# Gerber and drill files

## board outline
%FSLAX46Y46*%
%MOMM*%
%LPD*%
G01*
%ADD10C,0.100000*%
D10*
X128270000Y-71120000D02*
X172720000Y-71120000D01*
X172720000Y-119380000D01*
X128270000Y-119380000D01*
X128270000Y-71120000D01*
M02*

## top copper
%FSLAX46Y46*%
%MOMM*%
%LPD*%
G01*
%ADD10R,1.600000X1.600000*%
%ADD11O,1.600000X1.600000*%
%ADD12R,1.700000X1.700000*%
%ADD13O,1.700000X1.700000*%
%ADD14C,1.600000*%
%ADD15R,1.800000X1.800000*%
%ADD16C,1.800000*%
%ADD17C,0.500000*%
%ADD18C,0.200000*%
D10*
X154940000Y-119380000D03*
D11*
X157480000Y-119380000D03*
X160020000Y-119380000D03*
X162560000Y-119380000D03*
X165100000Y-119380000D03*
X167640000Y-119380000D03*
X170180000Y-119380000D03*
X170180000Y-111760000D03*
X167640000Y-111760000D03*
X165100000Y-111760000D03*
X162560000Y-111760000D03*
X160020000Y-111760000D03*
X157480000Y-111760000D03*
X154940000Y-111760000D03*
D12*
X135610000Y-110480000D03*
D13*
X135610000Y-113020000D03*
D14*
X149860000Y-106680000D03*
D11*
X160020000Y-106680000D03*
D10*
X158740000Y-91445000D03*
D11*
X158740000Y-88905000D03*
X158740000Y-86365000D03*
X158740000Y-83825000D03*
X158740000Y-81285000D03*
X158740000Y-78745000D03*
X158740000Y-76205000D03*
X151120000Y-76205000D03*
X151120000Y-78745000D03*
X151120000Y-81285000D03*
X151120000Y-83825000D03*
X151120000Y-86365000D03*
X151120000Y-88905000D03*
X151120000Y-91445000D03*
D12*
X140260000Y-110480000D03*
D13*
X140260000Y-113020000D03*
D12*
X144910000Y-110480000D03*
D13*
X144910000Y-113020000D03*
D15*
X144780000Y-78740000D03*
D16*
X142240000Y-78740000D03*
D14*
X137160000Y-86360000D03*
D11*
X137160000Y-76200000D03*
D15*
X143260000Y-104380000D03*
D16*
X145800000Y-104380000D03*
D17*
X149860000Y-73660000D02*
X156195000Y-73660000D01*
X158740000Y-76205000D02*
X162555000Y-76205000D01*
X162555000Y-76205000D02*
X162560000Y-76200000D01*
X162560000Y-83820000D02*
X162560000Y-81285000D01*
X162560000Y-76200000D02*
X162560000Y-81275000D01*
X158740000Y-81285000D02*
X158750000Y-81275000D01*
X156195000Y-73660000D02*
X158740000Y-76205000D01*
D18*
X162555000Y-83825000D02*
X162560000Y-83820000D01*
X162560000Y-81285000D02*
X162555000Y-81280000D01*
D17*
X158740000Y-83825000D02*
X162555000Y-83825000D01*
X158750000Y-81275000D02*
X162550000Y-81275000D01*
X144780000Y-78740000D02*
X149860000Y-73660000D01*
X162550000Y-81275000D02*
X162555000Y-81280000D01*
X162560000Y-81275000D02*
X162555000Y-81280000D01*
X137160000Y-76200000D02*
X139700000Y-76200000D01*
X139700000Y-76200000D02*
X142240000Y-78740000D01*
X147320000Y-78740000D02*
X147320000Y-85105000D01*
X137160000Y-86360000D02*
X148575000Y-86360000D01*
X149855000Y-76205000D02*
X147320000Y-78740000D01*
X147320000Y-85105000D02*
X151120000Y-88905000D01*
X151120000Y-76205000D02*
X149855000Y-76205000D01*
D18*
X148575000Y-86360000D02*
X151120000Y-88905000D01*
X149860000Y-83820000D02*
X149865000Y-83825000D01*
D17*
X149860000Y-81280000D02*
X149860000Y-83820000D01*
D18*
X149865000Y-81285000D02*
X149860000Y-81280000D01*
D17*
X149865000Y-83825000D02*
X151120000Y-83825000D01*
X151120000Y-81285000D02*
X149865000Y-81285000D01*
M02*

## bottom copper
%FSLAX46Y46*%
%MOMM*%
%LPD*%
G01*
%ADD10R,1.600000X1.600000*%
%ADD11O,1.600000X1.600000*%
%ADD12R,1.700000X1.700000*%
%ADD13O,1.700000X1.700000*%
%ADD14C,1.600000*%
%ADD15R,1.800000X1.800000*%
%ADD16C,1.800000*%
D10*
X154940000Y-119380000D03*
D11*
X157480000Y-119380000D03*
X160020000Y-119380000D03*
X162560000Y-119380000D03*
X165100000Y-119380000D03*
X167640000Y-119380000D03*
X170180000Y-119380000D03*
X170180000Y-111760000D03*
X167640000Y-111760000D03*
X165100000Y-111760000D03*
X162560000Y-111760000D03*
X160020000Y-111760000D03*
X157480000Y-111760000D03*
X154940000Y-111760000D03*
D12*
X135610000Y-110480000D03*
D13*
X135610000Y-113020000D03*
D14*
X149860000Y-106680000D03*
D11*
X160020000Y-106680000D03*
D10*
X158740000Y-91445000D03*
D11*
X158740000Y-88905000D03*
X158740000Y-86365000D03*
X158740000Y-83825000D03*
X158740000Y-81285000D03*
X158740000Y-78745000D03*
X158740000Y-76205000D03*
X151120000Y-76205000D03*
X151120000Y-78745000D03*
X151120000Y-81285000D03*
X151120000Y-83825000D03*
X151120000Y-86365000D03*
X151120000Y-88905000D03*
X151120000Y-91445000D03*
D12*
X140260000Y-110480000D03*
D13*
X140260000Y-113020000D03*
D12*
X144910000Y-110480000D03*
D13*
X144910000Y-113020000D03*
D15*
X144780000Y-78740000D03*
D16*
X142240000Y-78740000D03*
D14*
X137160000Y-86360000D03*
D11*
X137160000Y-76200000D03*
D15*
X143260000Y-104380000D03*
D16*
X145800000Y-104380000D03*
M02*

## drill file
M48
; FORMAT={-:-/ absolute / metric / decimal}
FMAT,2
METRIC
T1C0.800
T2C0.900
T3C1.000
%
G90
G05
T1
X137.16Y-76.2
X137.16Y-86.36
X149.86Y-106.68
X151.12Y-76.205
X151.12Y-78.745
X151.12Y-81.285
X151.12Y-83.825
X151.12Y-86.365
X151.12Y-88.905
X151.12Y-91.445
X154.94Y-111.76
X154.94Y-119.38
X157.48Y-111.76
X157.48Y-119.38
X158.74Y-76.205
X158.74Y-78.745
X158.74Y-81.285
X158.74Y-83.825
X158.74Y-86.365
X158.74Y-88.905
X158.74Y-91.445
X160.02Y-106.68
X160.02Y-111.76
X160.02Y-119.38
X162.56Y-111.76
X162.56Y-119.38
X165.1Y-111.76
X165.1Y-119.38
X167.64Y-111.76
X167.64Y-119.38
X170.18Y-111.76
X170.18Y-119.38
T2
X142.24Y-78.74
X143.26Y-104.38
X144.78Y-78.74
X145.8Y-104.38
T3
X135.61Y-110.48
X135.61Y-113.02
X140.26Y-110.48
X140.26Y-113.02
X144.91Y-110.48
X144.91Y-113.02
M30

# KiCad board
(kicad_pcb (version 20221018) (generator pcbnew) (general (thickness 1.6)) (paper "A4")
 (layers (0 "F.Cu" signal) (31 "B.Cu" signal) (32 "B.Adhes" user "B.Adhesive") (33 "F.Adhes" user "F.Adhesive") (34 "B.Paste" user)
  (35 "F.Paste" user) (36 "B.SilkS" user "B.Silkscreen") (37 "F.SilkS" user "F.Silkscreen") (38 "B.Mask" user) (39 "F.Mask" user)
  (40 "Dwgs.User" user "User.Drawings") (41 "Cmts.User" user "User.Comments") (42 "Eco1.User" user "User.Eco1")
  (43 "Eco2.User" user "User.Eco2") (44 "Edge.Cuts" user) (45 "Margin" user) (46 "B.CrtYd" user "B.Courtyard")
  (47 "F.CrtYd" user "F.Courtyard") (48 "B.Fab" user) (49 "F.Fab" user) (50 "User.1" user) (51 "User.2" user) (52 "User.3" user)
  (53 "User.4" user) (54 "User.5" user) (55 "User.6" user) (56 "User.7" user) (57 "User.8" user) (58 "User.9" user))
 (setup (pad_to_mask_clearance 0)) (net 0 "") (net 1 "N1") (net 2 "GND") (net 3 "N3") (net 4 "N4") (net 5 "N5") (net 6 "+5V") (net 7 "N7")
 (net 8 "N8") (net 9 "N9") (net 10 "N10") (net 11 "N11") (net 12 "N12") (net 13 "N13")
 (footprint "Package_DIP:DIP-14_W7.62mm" (layer "F.Cu") (at 154.94 119.38 90)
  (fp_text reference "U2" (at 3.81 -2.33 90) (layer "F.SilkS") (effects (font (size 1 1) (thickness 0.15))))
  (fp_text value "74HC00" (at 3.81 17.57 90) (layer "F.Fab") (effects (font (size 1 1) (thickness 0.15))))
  (pad "1" thru_hole rect (at 0 0 90) (size 1.6 1.6) (drill 0.8) (layers "*.Cu" "*.Mask") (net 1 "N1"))
  (pad "2" thru_hole oval (at 0 2.54 90) (size 1.6 1.6) (drill 0.8) (layers "*.Cu" "*.Mask") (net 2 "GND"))
  (pad "3" thru_hole oval (at 0 5.08 90) (size 1.6 1.6) (drill 0.8) (layers "*.Cu" "*.Mask") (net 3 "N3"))
  (pad "4" thru_hole oval (at 0 7.62 90) (size 1.6 1.6) (drill 0.8) (layers "*.Cu" "*.Mask") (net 2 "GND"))
  (pad "5" thru_hole oval (at 0 10.16 90) (size 1.6 1.6) (drill 0.8) (layers "*.Cu" "*.Mask") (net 2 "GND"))
  (pad "6" thru_hole oval (at 0 12.7 90) (size 1.6 1.6) (drill 0.8) (layers "*.Cu" "*.Mask") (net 1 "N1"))
  (pad "7" thru_hole oval (at 0 15.24 90) (size 1.6 1.6) (drill 0.8) (layers "*.Cu" "*.Mask") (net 2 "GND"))
  (pad "8" thru_hole oval (at 7.62 15.24 90) (size 1.6 1.6) (drill 0.8) (layers "*.Cu" "*.Mask") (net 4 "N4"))
  (pad "9" thru_hole oval (at 7.62 12.7 90) (size 1.6 1.6) (drill 0.8) (layers "*.Cu" "*.Mask") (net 1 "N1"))
  (pad "10" thru_hole oval (at 7.62 10.16 90) (size 1.6 1.6) (drill 0.8) (layers "*.Cu" "*.Mask") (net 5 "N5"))
  (pad "11" thru_hole oval (at 7.62 7.62 90) (size 1.6 1.6) (drill 0.8) (layers "*.Cu" "*.Mask") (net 5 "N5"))
  (pad "12" thru_hole oval (at 7.62 5.08 90) (size 1.6 1.6) (drill 0.8) (layers "*.Cu" "*.Mask") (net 3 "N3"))
  (pad "13" thru_hole oval (at 7.62 2.54 90) (size 1.6 1.6) (drill 0.8) (layers "*.Cu" "*.Mask") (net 4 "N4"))
  (pad "14" thru_hole oval (at 7.62 0 90) (size 1.6 1.6) (drill 0.8) (layers "*.Cu" "*.Mask") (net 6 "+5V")))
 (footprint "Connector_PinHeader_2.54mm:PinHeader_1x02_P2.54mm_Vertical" (layer "F.Cu") (at 135.61 110.48)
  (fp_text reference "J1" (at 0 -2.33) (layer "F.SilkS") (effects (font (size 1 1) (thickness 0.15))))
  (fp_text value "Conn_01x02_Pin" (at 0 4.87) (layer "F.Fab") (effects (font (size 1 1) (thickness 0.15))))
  (pad "1" thru_hole rect (at 0 0) (size 1.7 1.7) (drill 1) (layers "*.Cu" "*.Mask") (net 6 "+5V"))
  (pad "2" thru_hole oval (at 0 2.54) (size 1.7 1.7) (drill 1) (layers "*.Cu" "*.Mask") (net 2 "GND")))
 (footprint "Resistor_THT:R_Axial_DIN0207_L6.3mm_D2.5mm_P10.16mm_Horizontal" (layer "F.Cu") (at 149.86 106.68)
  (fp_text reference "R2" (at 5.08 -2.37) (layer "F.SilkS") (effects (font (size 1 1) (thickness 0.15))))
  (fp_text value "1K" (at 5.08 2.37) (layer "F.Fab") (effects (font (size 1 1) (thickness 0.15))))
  (pad "1" thru_hole circle (at 0 0) (size 1.6 1.6) (drill 0.8) (layers "*.Cu" "*.Mask") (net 4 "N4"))
  (pad "2" thru_hole oval (at 10.16 0) (size 1.6 1.6) (drill 0.8) (layers "*.Cu" "*.Mask") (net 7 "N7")))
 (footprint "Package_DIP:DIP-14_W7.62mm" (layer "F.Cu") (at 158.74 91.445 180)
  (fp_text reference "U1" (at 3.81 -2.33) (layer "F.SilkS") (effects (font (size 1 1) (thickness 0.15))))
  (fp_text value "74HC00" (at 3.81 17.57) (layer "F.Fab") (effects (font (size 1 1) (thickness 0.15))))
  (pad "1" thru_hole rect (at 0 0 180) (size 1.6 1.6) (drill 0.8) (layers "*.Cu" "*.Mask") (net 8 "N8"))
  (pad "2" thru_hole oval (at 0 2.54 180) (size 1.6 1.6) (drill 0.8) (layers "*.Cu" "*.Mask") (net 2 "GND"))
  (pad "3" thru_hole oval (at 0 5.08 180) (size 1.6 1.6) (drill 0.8) (layers "*.Cu" "*.Mask") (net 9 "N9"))
  (pad "4" thru_hole oval (at 0 7.62 180) (size 1.6 1.6) (drill 0.8) (layers "*.Cu" "*.Mask") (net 2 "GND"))
  (pad "5" thru_hole oval (at 0 10.16 180) (size 1.6 1.6) (drill 0.8) (layers "*.Cu" "*.Mask") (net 2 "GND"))
  (pad "6" thru_hole oval (at 0 12.7 180) (size 1.6 1.6) (drill 0.8) (layers "*.Cu" "*.Mask") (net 8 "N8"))
  (pad "7" thru_hole oval (at 0 15.24 180) (size 1.6 1.6) (drill 0.8) (layers "*.Cu" "*.Mask") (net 2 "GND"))
  (pad "8" thru_hole oval (at 7.62 15.24 180) (size 1.6 1.6) (drill 0.8) (layers "*.Cu" "*.Mask") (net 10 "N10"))
  (pad "9" thru_hole oval (at 7.62 12.7 180) (size 1.6 1.6) (drill 0.8) (layers "*.Cu" "*.Mask") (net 8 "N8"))
  (pad "10" thru_hole oval (at 7.62 10.16 180) (size 1.6 1.6) (drill 0.8) (layers "*.Cu" "*.Mask") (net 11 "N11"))
  (pad "11" thru_hole oval (at 7.62 7.62 180) (size 1.6 1.6) (drill 0.8) (layers "*.Cu" "*.Mask") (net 11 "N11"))
  (pad "12" thru_hole oval (at 7.62 5.08 180) (size 1.6 1.6) (drill 0.8) (layers "*.Cu" "*.Mask") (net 9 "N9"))
  (pad "13" thru_hole oval (at 7.62 2.54 180) (size 1.6 1.6) (drill 0.8) (layers "*.Cu" "*.Mask") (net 10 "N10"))
  (pad "14" thru_hole oval (at 7.62 0 180) (size 1.6 1.6) (drill 0.8) (layers "*.Cu" "*.Mask") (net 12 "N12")))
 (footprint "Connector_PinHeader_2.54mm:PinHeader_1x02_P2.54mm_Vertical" (layer "F.Cu") (at 140.26 110.48)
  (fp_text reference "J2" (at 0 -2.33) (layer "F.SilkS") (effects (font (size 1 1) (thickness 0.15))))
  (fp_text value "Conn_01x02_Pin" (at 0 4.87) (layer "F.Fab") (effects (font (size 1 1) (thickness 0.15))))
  (pad "1" thru_hole rect (at 0 0) (size 1.7 1.7) (drill 1) (layers "*.Cu" "*.Mask") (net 6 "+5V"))
  (pad "2" thru_hole oval (at 0 2.54) (size 1.7 1.7) (drill 1) (layers "*.Cu" "*.Mask") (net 2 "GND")))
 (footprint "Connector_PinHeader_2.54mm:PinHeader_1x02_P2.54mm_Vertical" (layer "F.Cu") (at 144.91 110.48)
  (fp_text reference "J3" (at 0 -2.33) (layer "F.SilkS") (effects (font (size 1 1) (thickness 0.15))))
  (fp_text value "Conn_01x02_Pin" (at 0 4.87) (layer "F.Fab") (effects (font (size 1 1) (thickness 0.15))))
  (pad "1" thru_hole rect (at 0 0) (size 1.7 1.7) (drill 1) (layers "*.Cu" "*.Mask") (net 6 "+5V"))
  (pad "2" thru_hole oval (at 0 2.54) (size 1.7 1.7) (drill 1) (layers "*.Cu" "*.Mask") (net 2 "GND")))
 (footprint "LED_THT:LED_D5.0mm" (layer "F.Cu") (at 144.78 78.74 180)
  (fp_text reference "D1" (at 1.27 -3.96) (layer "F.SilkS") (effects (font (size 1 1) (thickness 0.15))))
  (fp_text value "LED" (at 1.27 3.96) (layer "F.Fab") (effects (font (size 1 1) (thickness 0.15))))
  (pad "1" thru_hole rect (at 0 0 180) (size 1.8 1.8) (drill 0.9) (layers "*.Cu" "*.Mask") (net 2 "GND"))
  (pad "2" thru_hole circle (at 2.54 0 180) (size 1.8 1.8) (drill 0.9) (layers "*.Cu" "*.Mask") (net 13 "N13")))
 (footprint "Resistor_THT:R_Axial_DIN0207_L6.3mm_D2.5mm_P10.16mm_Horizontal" (layer "F.Cu") (at 137.16 86.36 90)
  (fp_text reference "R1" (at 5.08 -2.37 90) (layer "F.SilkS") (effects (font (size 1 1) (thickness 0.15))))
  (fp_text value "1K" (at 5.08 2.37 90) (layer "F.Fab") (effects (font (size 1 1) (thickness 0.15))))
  (pad "1" thru_hole circle (at 0 0 90) (size 1.6 1.6) (drill 0.8) (layers "*.Cu" "*.Mask") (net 10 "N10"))
  (pad "2" thru_hole oval (at 10.16 0 90) (size 1.6 1.6) (drill 0.8) (layers "*.Cu" "*.Mask") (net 13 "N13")))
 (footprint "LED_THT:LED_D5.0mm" (layer "F.Cu") (at 143.26 104.38)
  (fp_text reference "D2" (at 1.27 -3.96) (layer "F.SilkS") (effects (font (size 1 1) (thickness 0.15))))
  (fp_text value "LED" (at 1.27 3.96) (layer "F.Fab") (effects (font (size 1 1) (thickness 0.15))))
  (pad "1" thru_hole rect (at 0 0) (size 1.8 1.8) (drill 0.9) (layers "*.Cu" "*.Mask") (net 2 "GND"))
  (pad "2" thru_hole circle (at 2.54 0) (size 1.8 1.8) (drill 0.9) (layers "*.Cu" "*.Mask") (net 7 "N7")))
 (gr_rect (start 128.27 71.12) (end 172.72 119.38) (stroke (width 0.1) (type default)) (fill none) (layer "Edge.Cuts"))
 (segment (start 149.86 73.66) (end 156.195 73.66) (width 0.5) (layer "F.Cu") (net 2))
 (segment (start 158.74 76.205) (end 162.555 76.205) (width 0.5) (layer "F.Cu") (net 2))
 (segment (start 162.555 76.205) (end 162.56 76.2) (width 0.5) (layer "F.Cu") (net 2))
 (segment (start 162.56 83.82) (end 162.56 81.285) (width 0.5) (layer "F.Cu") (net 2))
 (segment (start 162.56 76.2) (end 162.56 81.275) (width 0.5) (layer "F.Cu") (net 2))
 (segment (start 158.74 81.285) (end 158.75 81.275) (width 0.5) (layer "F.Cu") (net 2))
 (segment (start 156.195 73.66) (end 158.74 76.205) (width 0.5) (layer "F.Cu") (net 2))
 (segment (start 162.555 83.825) (end 162.56 83.82) (width 0.2) (layer "F.Cu") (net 2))
 (segment (start 162.56 81.285) (end 162.555 81.28) (width 0.2) (layer "F.Cu") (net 2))
 (segment (start 158.74 83.825) (end 162.555 83.825) (width 0.5) (layer "F.Cu") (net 2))
 (segment (start 158.75 81.275) (end 162.55 81.275) (width 0.5) (layer "F.Cu") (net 2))
 (segment (start 144.78 78.74) (end 149.86 73.66) (width 0.5) (layer "F.Cu") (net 2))
 (segment (start 162.55 81.275) (end 162.555 81.28) (width 0.5) (layer "F.Cu") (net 2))
 (segment (start 162.56 81.275) (end 162.555 81.28) (width 0.5) (layer "F.Cu") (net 2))
 (segment (start 137.16 76.2) (end 139.7 76.2) (width 0.5) (layer "F.Cu") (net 13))
 (segment (start 139.7 76.2) (end 142.24 78.74) (width 0.5) (layer "F.Cu") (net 13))
 (segment (start 147.32 78.74) (end 147.32 85.105) (width 0.5) (layer "F.Cu") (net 10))
 (segment (start 137.16 86.36) (end 148.575 86.36) (width 0.5) (layer "F.Cu") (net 10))
 (segment (start 149.855 76.205) (end 147.32 78.74) (width 0.5) (layer "F.Cu") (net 10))
 (segment (start 147.32 85.105) (end 151.12 88.905) (width 0.5) (layer "F.Cu") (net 10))
 (segment (start 151.12 76.205) (end 149.855 76.205) (width 0.5) (layer "F.Cu") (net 10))
 (segment (start 148.575 86.36) (end 151.12 88.905) (width 0.2) (layer "F.Cu") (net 10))
 (segment (start 149.86 83.82) (end 149.865 83.825) (width 0.2) (layer "F.Cu") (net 11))
 (segment (start 149.86 81.28) (end 149.86 83.82) (width 0.5) (layer "F.Cu") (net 11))
 (segment (start 149.865 81.285) (end 149.86 81.28) (width 0.2) (layer "F.Cu") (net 11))
 (segment (start 149.865 83.825) (end 151.12 83.825) (width 0.5) (layer "F.Cu") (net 11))
 (segment (start 151.12 81.285) (end 149.865 81.285) (width 0.5) (layer "F.Cu") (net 11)))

